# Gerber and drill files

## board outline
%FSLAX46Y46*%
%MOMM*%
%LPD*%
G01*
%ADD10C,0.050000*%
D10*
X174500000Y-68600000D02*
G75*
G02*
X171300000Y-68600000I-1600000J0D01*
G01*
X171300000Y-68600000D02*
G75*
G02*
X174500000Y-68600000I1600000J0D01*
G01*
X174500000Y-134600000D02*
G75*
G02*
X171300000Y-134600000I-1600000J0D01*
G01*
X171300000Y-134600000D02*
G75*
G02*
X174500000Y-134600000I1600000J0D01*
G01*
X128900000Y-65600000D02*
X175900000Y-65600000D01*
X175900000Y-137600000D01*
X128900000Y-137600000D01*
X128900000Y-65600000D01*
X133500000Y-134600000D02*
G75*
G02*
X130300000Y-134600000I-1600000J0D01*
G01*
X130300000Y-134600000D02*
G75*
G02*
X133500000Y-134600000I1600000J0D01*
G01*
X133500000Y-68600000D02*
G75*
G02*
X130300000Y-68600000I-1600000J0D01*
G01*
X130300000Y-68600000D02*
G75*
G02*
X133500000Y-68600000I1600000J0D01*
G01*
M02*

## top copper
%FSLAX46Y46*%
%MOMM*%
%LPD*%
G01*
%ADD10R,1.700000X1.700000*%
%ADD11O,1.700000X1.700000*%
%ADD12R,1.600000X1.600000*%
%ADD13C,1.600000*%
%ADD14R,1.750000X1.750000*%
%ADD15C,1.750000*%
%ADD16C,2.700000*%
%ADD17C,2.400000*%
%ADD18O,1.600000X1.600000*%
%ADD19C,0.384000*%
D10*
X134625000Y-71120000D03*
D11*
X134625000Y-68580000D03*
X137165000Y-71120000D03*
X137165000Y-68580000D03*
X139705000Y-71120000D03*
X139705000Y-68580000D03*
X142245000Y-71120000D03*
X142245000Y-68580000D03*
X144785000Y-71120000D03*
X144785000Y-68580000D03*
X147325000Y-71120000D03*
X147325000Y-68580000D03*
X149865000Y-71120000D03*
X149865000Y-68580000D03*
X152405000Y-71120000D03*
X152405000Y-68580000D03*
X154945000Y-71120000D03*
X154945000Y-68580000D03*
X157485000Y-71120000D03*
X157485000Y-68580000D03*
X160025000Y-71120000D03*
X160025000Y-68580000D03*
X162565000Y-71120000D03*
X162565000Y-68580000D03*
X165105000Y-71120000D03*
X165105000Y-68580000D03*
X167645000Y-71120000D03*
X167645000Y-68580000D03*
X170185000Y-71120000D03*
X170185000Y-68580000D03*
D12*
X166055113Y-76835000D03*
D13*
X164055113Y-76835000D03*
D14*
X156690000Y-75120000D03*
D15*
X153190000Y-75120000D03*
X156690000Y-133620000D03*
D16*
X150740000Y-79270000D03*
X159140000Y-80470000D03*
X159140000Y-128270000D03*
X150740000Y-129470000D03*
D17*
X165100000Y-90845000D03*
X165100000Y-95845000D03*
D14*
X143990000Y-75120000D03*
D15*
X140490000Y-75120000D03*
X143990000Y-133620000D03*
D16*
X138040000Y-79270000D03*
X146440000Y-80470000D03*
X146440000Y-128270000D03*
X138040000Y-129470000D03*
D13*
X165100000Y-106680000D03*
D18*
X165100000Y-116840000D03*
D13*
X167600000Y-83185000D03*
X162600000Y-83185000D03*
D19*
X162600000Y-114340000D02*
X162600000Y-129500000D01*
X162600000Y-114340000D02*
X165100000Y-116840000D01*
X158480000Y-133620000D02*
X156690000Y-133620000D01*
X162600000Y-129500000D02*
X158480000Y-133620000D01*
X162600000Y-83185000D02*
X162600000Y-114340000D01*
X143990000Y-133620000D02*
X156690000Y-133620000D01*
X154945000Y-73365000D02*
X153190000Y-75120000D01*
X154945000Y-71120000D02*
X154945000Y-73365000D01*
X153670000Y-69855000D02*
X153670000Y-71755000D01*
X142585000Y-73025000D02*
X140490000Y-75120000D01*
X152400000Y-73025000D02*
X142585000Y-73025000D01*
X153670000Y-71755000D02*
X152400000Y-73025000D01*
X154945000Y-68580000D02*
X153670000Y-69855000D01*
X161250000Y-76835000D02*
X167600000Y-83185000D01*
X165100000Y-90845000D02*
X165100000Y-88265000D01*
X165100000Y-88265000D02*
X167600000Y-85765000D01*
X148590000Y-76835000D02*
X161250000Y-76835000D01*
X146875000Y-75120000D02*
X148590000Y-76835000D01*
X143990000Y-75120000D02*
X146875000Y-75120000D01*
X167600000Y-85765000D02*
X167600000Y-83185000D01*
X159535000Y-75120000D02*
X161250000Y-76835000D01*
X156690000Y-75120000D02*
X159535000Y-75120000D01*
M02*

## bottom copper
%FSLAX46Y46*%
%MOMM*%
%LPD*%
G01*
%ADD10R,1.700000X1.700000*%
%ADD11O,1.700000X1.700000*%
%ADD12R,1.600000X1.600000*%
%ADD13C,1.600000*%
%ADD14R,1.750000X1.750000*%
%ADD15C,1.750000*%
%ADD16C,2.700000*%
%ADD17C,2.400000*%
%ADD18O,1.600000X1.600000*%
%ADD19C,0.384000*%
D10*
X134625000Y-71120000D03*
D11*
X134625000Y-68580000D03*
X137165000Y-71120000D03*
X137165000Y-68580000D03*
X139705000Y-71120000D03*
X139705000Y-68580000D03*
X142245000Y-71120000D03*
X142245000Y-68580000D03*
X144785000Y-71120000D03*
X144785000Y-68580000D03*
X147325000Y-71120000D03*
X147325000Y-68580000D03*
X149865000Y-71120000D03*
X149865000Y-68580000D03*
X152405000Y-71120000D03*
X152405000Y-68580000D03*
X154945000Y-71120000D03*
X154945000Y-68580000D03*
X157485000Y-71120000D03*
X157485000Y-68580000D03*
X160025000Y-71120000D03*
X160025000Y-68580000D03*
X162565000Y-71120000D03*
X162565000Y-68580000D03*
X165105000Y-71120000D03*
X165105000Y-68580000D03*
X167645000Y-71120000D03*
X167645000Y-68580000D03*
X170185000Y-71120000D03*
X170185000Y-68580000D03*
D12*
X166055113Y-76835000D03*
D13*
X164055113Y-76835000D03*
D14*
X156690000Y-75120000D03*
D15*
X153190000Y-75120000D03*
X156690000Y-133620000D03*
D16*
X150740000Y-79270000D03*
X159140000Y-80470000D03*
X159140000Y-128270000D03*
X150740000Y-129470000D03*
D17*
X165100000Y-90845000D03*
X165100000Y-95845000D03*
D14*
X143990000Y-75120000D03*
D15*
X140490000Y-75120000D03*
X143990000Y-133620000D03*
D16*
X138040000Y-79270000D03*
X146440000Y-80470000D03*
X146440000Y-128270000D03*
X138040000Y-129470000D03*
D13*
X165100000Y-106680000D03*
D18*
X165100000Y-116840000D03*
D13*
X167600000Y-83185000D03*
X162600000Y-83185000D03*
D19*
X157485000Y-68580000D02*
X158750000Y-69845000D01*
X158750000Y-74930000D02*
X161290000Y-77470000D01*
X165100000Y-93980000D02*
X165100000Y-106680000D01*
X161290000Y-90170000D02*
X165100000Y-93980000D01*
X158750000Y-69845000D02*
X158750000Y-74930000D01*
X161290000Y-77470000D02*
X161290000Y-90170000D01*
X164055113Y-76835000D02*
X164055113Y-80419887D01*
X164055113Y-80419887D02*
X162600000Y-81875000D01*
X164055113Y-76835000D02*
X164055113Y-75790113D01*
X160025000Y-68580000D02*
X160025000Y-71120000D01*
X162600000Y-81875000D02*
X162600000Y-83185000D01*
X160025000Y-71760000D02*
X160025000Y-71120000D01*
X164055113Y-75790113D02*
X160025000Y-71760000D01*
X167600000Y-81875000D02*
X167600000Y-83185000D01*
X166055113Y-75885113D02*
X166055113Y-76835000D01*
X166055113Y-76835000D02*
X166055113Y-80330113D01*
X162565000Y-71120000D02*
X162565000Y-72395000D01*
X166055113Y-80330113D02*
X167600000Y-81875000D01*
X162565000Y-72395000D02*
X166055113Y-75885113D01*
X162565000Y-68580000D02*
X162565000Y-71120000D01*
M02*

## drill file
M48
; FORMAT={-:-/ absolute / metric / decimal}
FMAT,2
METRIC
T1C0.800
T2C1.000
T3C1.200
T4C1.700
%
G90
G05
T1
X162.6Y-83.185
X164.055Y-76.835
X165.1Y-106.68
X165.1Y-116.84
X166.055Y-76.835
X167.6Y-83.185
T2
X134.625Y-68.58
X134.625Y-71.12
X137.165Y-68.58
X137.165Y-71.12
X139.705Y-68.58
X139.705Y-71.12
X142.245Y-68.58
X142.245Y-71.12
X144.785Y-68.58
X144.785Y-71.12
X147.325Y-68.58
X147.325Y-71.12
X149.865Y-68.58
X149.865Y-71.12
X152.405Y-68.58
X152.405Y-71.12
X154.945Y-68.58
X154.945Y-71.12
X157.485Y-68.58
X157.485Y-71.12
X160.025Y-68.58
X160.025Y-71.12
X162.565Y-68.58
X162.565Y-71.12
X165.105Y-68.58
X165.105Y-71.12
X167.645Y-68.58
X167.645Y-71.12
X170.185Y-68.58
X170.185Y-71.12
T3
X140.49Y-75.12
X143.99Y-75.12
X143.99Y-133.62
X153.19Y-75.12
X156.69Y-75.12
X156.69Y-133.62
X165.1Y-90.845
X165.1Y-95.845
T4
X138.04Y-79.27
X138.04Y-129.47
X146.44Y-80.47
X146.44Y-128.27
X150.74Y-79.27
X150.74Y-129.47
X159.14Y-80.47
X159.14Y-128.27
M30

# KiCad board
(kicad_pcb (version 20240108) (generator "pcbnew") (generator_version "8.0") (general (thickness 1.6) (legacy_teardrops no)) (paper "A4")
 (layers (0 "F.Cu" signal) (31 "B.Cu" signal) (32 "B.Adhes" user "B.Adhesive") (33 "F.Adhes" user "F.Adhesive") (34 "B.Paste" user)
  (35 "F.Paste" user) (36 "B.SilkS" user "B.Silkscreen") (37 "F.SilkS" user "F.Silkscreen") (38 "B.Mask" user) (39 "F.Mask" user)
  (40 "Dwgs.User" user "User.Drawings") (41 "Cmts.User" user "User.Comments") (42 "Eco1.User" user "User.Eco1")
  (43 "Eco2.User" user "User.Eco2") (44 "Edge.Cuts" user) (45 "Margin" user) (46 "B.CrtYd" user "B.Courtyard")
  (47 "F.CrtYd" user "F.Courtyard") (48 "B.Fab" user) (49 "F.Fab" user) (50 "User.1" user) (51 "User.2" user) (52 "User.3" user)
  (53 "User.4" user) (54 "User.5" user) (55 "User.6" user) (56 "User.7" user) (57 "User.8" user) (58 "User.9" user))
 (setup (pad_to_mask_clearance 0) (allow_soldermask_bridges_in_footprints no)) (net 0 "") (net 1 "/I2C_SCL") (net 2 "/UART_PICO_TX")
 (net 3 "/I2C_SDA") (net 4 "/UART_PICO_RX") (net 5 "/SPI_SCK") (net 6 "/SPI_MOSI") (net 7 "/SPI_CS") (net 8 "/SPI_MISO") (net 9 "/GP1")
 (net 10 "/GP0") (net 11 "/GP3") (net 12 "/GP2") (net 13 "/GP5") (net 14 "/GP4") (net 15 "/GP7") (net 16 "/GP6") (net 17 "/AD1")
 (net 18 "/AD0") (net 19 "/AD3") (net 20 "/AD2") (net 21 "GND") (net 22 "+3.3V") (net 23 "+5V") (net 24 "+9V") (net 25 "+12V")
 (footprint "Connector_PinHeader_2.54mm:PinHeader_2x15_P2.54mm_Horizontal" (layer "F.Cu") (at 134.625 71.12 90)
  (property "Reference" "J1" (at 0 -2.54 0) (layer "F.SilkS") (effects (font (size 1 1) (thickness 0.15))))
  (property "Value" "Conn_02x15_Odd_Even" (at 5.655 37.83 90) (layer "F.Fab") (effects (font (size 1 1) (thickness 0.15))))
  (pad "1" thru_hole rect (at 0 0 90) (size 1.7 1.7) (drill 1) (layers "*.Cu" "*.Mask") (remove_unused_layers no) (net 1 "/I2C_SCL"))
  (pad "2" thru_hole oval (at 2.54 0 90) (size 1.7 1.7) (drill 1) (layers "*.Cu" "*.Mask") (remove_unused_layers no) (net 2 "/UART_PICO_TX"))
  (pad "3" thru_hole oval (at 0 2.54 90) (size 1.7 1.7) (drill 1) (layers "*.Cu" "*.Mask") (remove_unused_layers no) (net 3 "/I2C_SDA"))
  (pad "4" thru_hole oval (at 2.54 2.54 90) (size 1.7 1.7) (drill 1) (layers "*.Cu" "*.Mask") (remove_unused_layers no)
   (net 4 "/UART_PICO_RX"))
  (pad "5" thru_hole oval (at 0 5.08 90) (size 1.7 1.7) (drill 1) (layers "*.Cu" "*.Mask") (remove_unused_layers no) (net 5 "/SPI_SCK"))
  (pad "6" thru_hole oval (at 2.54 5.08 90) (size 1.7 1.7) (drill 1) (layers "*.Cu" "*.Mask") (remove_unused_layers no) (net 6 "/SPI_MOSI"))
  (pad "7" thru_hole oval (at 0 7.62 90) (size 1.7 1.7) (drill 1) (layers "*.Cu" "*.Mask") (remove_unused_layers no) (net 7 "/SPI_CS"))
  (pad "8" thru_hole oval (at 2.54 7.62 90) (size 1.7 1.7) (drill 1) (layers "*.Cu" "*.Mask") (remove_unused_layers no) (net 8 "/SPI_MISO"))
  (pad "9" thru_hole oval (at 0 10.16 90) (size 1.7 1.7) (drill 1) (layers "*.Cu" "*.Mask") (remove_unused_layers no) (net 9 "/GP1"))
  (pad "10" thru_hole oval (at 2.54 10.16 90) (size 1.7 1.7) (drill 1) (layers "*.Cu" "*.Mask") (remove_unused_layers no) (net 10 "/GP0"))
  (pad "11" thru_hole oval (at 0 12.7 90) (size 1.7 1.7) (drill 1) (layers "*.Cu" "*.Mask") (remove_unused_layers no) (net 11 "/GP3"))
  (pad "12" thru_hole oval (at 2.54 12.7 90) (size 1.7 1.7) (drill 1) (layers "*.Cu" "*.Mask") (remove_unused_layers no) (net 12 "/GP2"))
  (pad "13" thru_hole oval (at 0 15.24 90) (size 1.7 1.7) (drill 1) (layers "*.Cu" "*.Mask") (remove_unused_layers no) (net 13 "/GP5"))
  (pad "14" thru_hole oval (at 2.54 15.24 90) (size 1.7 1.7) (drill 1) (layers "*.Cu" "*.Mask") (remove_unused_layers no) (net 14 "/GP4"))
  (pad "15" thru_hole oval (at 0 17.78 90) (size 1.7 1.7) (drill 1) (layers "*.Cu" "*.Mask") (remove_unused_layers no) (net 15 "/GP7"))
  (pad "16" thru_hole oval (at 2.54 17.78 90) (size 1.7 1.7) (drill 1) (layers "*.Cu" "*.Mask") (remove_unused_layers no) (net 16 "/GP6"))
  (pad "17" thru_hole oval (at 0 20.32 90) (size 1.7 1.7) (drill 1) (layers "*.Cu" "*.Mask") (remove_unused_layers no) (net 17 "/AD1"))
  (pad "18" thru_hole oval (at 2.54 20.32 90) (size 1.7 1.7) (drill 1) (layers "*.Cu" "*.Mask") (remove_unused_layers no) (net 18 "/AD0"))
  (pad "19" thru_hole oval (at 0 22.86 90) (size 1.7 1.7) (drill 1) (layers "*.Cu" "*.Mask") (remove_unused_layers no) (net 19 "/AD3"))
  (pad "20" thru_hole oval (at 2.54 22.86 90) (size 1.7 1.7) (drill 1) (layers "*.Cu" "*.Mask") (remove_unused_layers no) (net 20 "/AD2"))
  (pad "21" thru_hole oval (at 0 25.4 90) (size 1.7 1.7) (drill 1) (layers "*.Cu" "*.Mask") (remove_unused_layers no) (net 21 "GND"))
  (pad "22" thru_hole oval (at 2.54 25.4 90) (size 1.7 1.7) (drill 1) (layers "*.Cu" "*.Mask") (remove_unused_layers no) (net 21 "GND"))
  (pad "23" thru_hole oval (at 0 27.94 90) (size 1.7 1.7) (drill 1) (layers "*.Cu" "*.Mask") (remove_unused_layers no) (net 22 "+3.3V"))
  (pad "24" thru_hole oval (at 2.54 27.94 90) (size 1.7 1.7) (drill 1) (layers "*.Cu" "*.Mask") (remove_unused_layers no) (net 22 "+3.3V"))
  (pad "25" thru_hole oval (at 0 30.48 90) (size 1.7 1.7) (drill 1) (layers "*.Cu" "*.Mask") (remove_unused_layers no) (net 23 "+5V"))
  (pad "26" thru_hole oval (at 2.54 30.48 90) (size 1.7 1.7) (drill 1) (layers "*.Cu" "*.Mask") (remove_unused_layers no) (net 23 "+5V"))
  (pad "27" thru_hole oval (at 0 33.02 90) (size 1.7 1.7) (drill 1) (layers "*.Cu" "*.Mask") (remove_unused_layers no) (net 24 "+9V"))
  (pad "28" thru_hole oval (at 2.54 33.02 90) (size 1.7 1.7) (drill 1) (layers "*.Cu" "*.Mask") (remove_unused_layers no) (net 24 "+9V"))
  (pad "29" thru_hole oval (at 0 35.56 90) (size 1.7 1.7) (drill 1) (layers "*.Cu" "*.Mask") (remove_unused_layers no) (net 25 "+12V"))
  (pad "30" thru_hole oval (at 2.54 35.56 90) (size 1.7 1.7) (drill 1) (layers "*.Cu" "*.Mask") (remove_unused_layers no) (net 25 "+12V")))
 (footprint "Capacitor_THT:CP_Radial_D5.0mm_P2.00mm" (layer "F.Cu") (at 166.055113 76.835 180)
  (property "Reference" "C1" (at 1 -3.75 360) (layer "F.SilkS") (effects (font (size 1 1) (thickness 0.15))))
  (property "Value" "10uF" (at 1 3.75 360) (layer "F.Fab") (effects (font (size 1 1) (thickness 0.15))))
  (pad "1" thru_hole rect (at 0 0 180) (size 1.6 1.6) (drill 0.8) (layers "*.Cu" "*.Mask") (remove_unused_layers no) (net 22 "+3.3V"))
  (pad "2" thru_hole circle (at 2 0 180) (size 1.6 1.6) (drill 0.8) (layers "*.Cu" "*.Mask") (remove_unused_layers no) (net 21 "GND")))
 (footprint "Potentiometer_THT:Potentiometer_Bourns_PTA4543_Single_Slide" (layer "F.Cu") (at 156.69 75.12 -90)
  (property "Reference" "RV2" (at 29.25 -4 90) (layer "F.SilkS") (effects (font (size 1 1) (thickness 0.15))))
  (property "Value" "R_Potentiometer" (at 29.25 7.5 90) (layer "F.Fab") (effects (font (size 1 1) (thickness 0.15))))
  (pad "1" thru_hole rect (at 0 0 270) (size 1.75 1.75) (drill 1.2) (layers "*.Cu" "*.Mask") (remove_unused_layers no) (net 22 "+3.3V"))
  (pad "2" thru_hole circle (at 0 3.5 270) (size 1.75 1.75) (drill 1.2) (layers "*.Cu" "*.Mask") (remove_unused_layers no) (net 17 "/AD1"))
  (pad "3" thru_hole circle (at 58.5 0 270) (size 1.75 1.75) (drill 1.2) (layers "*.Cu" "*.Mask") (remove_unused_layers no) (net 21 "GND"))
  (pad "MP" thru_hole circle (at 4.15 5.95 270) (size 2.7 2.7) (drill 1.7) (layers "*.Cu" "*.Mask") (remove_unused_layers no))
  (pad "MP" thru_hole circle (at 5.35 -2.45 270) (size 2.7 2.7) (drill 1.7) (layers "*.Cu" "*.Mask") (remove_unused_layers no))
  (pad "MP" thru_hole circle (at 53.15 -2.45 270) (size 2.7 2.7) (drill 1.7) (layers "*.Cu" "*.Mask") (remove_unused_layers no))
  (pad "MP" thru_hole circle (at 54.35 5.95 270) (size 2.7 2.7) (drill 1.7) (layers "*.Cu" "*.Mask") (remove_unused_layers no)))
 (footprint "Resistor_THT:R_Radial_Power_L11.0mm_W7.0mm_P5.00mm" (layer "F.Cu") (at 165.1 90.845 -90)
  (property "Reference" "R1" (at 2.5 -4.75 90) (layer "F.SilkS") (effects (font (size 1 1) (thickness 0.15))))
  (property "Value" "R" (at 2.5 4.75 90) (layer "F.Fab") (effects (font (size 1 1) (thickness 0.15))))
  (pad "1" thru_hole circle (at 0 0 270) (size 2.4 2.4) (drill 1.2) (layers "*.Cu" "*.Mask") (remove_unused_layers no) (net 22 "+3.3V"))
  (pad "2" thru_hole circle (at 5 0 270) (size 2.4 2.4) (drill 1.2) (layers "*.Cu" "*.Mask") (remove_unused_layers no) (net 20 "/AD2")))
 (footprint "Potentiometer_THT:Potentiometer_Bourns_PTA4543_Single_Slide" (layer "F.Cu") (at 143.99 75.12 -90)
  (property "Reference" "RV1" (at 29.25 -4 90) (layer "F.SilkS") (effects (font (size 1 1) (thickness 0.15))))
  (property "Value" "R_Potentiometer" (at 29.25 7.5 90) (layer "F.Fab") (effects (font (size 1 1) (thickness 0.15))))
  (pad "1" thru_hole rect (at 0 0 270) (size 1.75 1.75) (drill 1.2) (layers "*.Cu" "*.Mask") (remove_unused_layers no) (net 22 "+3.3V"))
  (pad "2" thru_hole circle (at 0 3.5 270) (size 1.75 1.75) (drill 1.2) (layers "*.Cu" "*.Mask") (remove_unused_layers no) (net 18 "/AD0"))
  (pad "3" thru_hole circle (at 58.5 0 270) (size 1.75 1.75) (drill 1.2) (layers "*.Cu" "*.Mask") (remove_unused_layers no) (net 21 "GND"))
  (pad "MP" thru_hole circle (at 4.15 5.95 270) (size 2.7 2.7) (drill 1.7) (layers "*.Cu" "*.Mask") (remove_unused_layers no))
  (pad "MP" thru_hole circle (at 5.35 -2.45 270) (size 2.7 2.7) (drill 1.7) (layers "*.Cu" "*.Mask") (remove_unused_layers no))
  (pad "MP" thru_hole circle (at 53.15 -2.45 270) (size 2.7 2.7) (drill 1.7) (layers "*.Cu" "*.Mask") (remove_unused_layers no))
  (pad "MP" thru_hole circle (at 54.35 5.95 270) (size 2.7 2.7) (drill 1.7) (layers "*.Cu" "*.Mask") (remove_unused_layers no)))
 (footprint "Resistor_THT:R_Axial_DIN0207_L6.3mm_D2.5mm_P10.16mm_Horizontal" (layer "F.Cu") (at 165.1 106.68 -90)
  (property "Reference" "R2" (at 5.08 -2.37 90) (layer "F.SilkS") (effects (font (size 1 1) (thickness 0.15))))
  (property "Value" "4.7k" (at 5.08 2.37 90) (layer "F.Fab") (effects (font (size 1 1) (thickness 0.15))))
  (pad "1" thru_hole circle (at 0 0 270) (size 1.6 1.6) (drill 0.8) (layers "*.Cu" "*.Mask") (remove_unused_layers no) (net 20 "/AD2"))
  (pad "2" thru_hole oval (at 10.16 0 270) (size 1.6 1.6) (drill 0.8) (layers "*.Cu" "*.Mask") (remove_unused_layers no) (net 21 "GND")))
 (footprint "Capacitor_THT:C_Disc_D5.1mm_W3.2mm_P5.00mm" (layer "F.Cu") (at 167.6 83.185 180)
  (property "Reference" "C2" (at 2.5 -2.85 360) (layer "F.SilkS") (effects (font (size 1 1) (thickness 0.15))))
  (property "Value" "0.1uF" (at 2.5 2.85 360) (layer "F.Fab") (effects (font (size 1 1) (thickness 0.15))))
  (pad "1" thru_hole circle (at 0 0 180) (size 1.6 1.6) (drill 0.8) (layers "*.Cu" "*.Mask") (remove_unused_layers no) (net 22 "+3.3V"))
  (pad "2" thru_hole circle (at 5 0 180) (size 1.6 1.6) (drill 0.8) (layers "*.Cu" "*.Mask") (remove_unused_layers no) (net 21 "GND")))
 (gr_circle (center 172.9 68.6) (end 172.9 70.2) (stroke (width 0.05) (type default)) (fill none) (layer "Edge.Cuts"))
 (gr_circle (center 172.9 134.6) (end 171.3 134.6) (stroke (width 0.05) (type default)) (fill none) (layer "Edge.Cuts"))
 (gr_rect (start 128.9 65.6) (end 175.9 137.6) (stroke (width 0.05) (type default)) (fill none) (layer "Edge.Cuts"))
 (gr_circle (center 131.9 134.6) (end 131.9 133) (stroke (width 0.05) (type default)) (fill none) (layer "Edge.Cuts"))
 (gr_circle (center 131.9 68.6) (end 133.5 68.6) (stroke (width 0.05) (type default)) (fill none) (layer "Edge.Cuts"))
 (segment (start 157.485 68.58) (end 158.75 69.845) (width 0.384) (layer "B.Cu") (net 20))
 (segment (start 158.75 74.93) (end 161.29 77.47) (width 0.384) (layer "B.Cu") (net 20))
 (segment (start 165.1 93.98) (end 165.1 106.68) (width 0.384) (layer "B.Cu") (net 20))
 (segment (start 161.29 90.17) (end 165.1 93.98) (width 0.384) (layer "B.Cu") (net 20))
 (segment (start 158.75 69.845) (end 158.75 74.93) (width 0.384) (layer "B.Cu") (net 20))
 (segment (start 161.29 77.47) (end 161.29 90.17) (width 0.384) (layer "B.Cu") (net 20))
 (segment (start 162.6 114.34) (end 162.6 129.5) (width 0.384) (layer "F.Cu") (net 21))
 (segment (start 162.6 114.34) (end 165.1 116.84) (width 0.384) (layer "F.Cu") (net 21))
 (segment (start 158.48 133.62) (end 156.69 133.62) (width 0.384) (layer "F.Cu") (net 21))
 (segment (start 162.6 129.5) (end 158.48 133.62) (width 0.384) (layer "F.Cu") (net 21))
 (segment (start 162.6 83.185) (end 162.6 114.34) (width 0.384) (layer "F.Cu") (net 21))
 (segment (start 143.99 133.62) (end 156.69 133.62) (width 0.384) (layer "F.Cu") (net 21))
 (segment (start 164.055113 76.835) (end 164.055113 80.419887) (width 0.384) (layer "B.Cu") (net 21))
 (segment (start 164.055113 80.419887) (end 162.6 81.875) (width 0.384) (layer "B.Cu") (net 21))
 (segment (start 164.055113 76.835) (end 164.055113 75.790113) (width 0.384) (layer "B.Cu") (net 21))
 (segment (start 160.025 68.58) (end 160.025 71.12) (width 0.384) (layer "B.Cu") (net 21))
 (segment (start 162.6 81.875) (end 162.6 83.185) (width 0.384) (layer "B.Cu") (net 21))
 (segment (start 160.025 71.76) (end 160.025 71.12) (width 0.384) (layer "B.Cu") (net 21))
 (segment (start 164.055113 75.790113) (end 160.025 71.76) (width 0.384) (layer "B.Cu") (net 21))
 (segment (start 154.945 73.365) (end 153.19 75.12) (width 0.384) (layer "F.Cu") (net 17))
 (segment (start 154.945 71.12) (end 154.945 73.365) (width 0.384) (layer "F.Cu") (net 17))
 (segment (start 153.67 69.855) (end 153.67 71.755) (width 0.384) (layer "F.Cu") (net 18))
 (segment (start 142.585 73.025) (end 140.49 75.12) (width 0.384) (layer "F.Cu") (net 18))
 (segment (start 152.4 73.025) (end 142.585 73.025) (width 0.384) (layer "F.Cu") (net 18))
 (segment (start 153.67 71.755) (end 152.4 73.025) (width 0.384) (layer "F.Cu") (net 18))
 (segment (start 154.945 68.58) (end 153.67 69.855) (width 0.384) (layer "F.Cu") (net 18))
 (segment (start 161.25 76.835) (end 167.6 83.185) (width 0.384) (layer "F.Cu") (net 22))
 (segment (start 165.1 90.845) (end 165.1 88.265) (width 0.384) (layer "F.Cu") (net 22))
 (segment (start 165.1 88.265) (end 167.6 85.765) (width 0.384) (layer "F.Cu") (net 22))
 (segment (start 148.59 76.835) (end 161.25 76.835) (width 0.384) (layer "F.Cu") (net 22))
 (segment (start 146.875 75.12) (end 148.59 76.835) (width 0.384) (layer "F.Cu") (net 22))
 (segment (start 143.99 75.12) (end 146.875 75.12) (width 0.384) (layer "F.Cu") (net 22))
 (segment (start 167.6 85.765) (end 167.6 83.185) (width 0.384) (layer "F.Cu") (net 22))
 (segment (start 159.535 75.12) (end 161.25 76.835) (width 0.384) (layer "F.Cu") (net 22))
 (segment (start 156.69 75.12) (end 159.535 75.12) (width 0.384) (layer "F.Cu") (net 22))
 (segment (start 167.6 81.875) (end 167.6 83.185) (width 0.384) (layer "B.Cu") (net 22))
 (segment (start 166.055113 75.885113) (end 166.055113 76.835) (width 0.384) (layer "B.Cu") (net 22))
 (segment (start 166.055113 76.835) (end 166.055113 80.330113) (width 0.384) (layer "B.Cu") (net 22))
 (segment (start 162.565 71.12) (end 162.565 72.395) (width 0.384) (layer "B.Cu") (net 22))
 (segment (start 166.055113 80.330113) (end 167.6 81.875) (width 0.384) (layer "B.Cu") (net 22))
 (segment (start 162.565 72.395) (end 166.055113 75.885113) (width 0.384) (layer "B.Cu") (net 22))
 (segment (start 162.565 68.58) (end 162.565 71.12) (width 0.384) (layer "B.Cu") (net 22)))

